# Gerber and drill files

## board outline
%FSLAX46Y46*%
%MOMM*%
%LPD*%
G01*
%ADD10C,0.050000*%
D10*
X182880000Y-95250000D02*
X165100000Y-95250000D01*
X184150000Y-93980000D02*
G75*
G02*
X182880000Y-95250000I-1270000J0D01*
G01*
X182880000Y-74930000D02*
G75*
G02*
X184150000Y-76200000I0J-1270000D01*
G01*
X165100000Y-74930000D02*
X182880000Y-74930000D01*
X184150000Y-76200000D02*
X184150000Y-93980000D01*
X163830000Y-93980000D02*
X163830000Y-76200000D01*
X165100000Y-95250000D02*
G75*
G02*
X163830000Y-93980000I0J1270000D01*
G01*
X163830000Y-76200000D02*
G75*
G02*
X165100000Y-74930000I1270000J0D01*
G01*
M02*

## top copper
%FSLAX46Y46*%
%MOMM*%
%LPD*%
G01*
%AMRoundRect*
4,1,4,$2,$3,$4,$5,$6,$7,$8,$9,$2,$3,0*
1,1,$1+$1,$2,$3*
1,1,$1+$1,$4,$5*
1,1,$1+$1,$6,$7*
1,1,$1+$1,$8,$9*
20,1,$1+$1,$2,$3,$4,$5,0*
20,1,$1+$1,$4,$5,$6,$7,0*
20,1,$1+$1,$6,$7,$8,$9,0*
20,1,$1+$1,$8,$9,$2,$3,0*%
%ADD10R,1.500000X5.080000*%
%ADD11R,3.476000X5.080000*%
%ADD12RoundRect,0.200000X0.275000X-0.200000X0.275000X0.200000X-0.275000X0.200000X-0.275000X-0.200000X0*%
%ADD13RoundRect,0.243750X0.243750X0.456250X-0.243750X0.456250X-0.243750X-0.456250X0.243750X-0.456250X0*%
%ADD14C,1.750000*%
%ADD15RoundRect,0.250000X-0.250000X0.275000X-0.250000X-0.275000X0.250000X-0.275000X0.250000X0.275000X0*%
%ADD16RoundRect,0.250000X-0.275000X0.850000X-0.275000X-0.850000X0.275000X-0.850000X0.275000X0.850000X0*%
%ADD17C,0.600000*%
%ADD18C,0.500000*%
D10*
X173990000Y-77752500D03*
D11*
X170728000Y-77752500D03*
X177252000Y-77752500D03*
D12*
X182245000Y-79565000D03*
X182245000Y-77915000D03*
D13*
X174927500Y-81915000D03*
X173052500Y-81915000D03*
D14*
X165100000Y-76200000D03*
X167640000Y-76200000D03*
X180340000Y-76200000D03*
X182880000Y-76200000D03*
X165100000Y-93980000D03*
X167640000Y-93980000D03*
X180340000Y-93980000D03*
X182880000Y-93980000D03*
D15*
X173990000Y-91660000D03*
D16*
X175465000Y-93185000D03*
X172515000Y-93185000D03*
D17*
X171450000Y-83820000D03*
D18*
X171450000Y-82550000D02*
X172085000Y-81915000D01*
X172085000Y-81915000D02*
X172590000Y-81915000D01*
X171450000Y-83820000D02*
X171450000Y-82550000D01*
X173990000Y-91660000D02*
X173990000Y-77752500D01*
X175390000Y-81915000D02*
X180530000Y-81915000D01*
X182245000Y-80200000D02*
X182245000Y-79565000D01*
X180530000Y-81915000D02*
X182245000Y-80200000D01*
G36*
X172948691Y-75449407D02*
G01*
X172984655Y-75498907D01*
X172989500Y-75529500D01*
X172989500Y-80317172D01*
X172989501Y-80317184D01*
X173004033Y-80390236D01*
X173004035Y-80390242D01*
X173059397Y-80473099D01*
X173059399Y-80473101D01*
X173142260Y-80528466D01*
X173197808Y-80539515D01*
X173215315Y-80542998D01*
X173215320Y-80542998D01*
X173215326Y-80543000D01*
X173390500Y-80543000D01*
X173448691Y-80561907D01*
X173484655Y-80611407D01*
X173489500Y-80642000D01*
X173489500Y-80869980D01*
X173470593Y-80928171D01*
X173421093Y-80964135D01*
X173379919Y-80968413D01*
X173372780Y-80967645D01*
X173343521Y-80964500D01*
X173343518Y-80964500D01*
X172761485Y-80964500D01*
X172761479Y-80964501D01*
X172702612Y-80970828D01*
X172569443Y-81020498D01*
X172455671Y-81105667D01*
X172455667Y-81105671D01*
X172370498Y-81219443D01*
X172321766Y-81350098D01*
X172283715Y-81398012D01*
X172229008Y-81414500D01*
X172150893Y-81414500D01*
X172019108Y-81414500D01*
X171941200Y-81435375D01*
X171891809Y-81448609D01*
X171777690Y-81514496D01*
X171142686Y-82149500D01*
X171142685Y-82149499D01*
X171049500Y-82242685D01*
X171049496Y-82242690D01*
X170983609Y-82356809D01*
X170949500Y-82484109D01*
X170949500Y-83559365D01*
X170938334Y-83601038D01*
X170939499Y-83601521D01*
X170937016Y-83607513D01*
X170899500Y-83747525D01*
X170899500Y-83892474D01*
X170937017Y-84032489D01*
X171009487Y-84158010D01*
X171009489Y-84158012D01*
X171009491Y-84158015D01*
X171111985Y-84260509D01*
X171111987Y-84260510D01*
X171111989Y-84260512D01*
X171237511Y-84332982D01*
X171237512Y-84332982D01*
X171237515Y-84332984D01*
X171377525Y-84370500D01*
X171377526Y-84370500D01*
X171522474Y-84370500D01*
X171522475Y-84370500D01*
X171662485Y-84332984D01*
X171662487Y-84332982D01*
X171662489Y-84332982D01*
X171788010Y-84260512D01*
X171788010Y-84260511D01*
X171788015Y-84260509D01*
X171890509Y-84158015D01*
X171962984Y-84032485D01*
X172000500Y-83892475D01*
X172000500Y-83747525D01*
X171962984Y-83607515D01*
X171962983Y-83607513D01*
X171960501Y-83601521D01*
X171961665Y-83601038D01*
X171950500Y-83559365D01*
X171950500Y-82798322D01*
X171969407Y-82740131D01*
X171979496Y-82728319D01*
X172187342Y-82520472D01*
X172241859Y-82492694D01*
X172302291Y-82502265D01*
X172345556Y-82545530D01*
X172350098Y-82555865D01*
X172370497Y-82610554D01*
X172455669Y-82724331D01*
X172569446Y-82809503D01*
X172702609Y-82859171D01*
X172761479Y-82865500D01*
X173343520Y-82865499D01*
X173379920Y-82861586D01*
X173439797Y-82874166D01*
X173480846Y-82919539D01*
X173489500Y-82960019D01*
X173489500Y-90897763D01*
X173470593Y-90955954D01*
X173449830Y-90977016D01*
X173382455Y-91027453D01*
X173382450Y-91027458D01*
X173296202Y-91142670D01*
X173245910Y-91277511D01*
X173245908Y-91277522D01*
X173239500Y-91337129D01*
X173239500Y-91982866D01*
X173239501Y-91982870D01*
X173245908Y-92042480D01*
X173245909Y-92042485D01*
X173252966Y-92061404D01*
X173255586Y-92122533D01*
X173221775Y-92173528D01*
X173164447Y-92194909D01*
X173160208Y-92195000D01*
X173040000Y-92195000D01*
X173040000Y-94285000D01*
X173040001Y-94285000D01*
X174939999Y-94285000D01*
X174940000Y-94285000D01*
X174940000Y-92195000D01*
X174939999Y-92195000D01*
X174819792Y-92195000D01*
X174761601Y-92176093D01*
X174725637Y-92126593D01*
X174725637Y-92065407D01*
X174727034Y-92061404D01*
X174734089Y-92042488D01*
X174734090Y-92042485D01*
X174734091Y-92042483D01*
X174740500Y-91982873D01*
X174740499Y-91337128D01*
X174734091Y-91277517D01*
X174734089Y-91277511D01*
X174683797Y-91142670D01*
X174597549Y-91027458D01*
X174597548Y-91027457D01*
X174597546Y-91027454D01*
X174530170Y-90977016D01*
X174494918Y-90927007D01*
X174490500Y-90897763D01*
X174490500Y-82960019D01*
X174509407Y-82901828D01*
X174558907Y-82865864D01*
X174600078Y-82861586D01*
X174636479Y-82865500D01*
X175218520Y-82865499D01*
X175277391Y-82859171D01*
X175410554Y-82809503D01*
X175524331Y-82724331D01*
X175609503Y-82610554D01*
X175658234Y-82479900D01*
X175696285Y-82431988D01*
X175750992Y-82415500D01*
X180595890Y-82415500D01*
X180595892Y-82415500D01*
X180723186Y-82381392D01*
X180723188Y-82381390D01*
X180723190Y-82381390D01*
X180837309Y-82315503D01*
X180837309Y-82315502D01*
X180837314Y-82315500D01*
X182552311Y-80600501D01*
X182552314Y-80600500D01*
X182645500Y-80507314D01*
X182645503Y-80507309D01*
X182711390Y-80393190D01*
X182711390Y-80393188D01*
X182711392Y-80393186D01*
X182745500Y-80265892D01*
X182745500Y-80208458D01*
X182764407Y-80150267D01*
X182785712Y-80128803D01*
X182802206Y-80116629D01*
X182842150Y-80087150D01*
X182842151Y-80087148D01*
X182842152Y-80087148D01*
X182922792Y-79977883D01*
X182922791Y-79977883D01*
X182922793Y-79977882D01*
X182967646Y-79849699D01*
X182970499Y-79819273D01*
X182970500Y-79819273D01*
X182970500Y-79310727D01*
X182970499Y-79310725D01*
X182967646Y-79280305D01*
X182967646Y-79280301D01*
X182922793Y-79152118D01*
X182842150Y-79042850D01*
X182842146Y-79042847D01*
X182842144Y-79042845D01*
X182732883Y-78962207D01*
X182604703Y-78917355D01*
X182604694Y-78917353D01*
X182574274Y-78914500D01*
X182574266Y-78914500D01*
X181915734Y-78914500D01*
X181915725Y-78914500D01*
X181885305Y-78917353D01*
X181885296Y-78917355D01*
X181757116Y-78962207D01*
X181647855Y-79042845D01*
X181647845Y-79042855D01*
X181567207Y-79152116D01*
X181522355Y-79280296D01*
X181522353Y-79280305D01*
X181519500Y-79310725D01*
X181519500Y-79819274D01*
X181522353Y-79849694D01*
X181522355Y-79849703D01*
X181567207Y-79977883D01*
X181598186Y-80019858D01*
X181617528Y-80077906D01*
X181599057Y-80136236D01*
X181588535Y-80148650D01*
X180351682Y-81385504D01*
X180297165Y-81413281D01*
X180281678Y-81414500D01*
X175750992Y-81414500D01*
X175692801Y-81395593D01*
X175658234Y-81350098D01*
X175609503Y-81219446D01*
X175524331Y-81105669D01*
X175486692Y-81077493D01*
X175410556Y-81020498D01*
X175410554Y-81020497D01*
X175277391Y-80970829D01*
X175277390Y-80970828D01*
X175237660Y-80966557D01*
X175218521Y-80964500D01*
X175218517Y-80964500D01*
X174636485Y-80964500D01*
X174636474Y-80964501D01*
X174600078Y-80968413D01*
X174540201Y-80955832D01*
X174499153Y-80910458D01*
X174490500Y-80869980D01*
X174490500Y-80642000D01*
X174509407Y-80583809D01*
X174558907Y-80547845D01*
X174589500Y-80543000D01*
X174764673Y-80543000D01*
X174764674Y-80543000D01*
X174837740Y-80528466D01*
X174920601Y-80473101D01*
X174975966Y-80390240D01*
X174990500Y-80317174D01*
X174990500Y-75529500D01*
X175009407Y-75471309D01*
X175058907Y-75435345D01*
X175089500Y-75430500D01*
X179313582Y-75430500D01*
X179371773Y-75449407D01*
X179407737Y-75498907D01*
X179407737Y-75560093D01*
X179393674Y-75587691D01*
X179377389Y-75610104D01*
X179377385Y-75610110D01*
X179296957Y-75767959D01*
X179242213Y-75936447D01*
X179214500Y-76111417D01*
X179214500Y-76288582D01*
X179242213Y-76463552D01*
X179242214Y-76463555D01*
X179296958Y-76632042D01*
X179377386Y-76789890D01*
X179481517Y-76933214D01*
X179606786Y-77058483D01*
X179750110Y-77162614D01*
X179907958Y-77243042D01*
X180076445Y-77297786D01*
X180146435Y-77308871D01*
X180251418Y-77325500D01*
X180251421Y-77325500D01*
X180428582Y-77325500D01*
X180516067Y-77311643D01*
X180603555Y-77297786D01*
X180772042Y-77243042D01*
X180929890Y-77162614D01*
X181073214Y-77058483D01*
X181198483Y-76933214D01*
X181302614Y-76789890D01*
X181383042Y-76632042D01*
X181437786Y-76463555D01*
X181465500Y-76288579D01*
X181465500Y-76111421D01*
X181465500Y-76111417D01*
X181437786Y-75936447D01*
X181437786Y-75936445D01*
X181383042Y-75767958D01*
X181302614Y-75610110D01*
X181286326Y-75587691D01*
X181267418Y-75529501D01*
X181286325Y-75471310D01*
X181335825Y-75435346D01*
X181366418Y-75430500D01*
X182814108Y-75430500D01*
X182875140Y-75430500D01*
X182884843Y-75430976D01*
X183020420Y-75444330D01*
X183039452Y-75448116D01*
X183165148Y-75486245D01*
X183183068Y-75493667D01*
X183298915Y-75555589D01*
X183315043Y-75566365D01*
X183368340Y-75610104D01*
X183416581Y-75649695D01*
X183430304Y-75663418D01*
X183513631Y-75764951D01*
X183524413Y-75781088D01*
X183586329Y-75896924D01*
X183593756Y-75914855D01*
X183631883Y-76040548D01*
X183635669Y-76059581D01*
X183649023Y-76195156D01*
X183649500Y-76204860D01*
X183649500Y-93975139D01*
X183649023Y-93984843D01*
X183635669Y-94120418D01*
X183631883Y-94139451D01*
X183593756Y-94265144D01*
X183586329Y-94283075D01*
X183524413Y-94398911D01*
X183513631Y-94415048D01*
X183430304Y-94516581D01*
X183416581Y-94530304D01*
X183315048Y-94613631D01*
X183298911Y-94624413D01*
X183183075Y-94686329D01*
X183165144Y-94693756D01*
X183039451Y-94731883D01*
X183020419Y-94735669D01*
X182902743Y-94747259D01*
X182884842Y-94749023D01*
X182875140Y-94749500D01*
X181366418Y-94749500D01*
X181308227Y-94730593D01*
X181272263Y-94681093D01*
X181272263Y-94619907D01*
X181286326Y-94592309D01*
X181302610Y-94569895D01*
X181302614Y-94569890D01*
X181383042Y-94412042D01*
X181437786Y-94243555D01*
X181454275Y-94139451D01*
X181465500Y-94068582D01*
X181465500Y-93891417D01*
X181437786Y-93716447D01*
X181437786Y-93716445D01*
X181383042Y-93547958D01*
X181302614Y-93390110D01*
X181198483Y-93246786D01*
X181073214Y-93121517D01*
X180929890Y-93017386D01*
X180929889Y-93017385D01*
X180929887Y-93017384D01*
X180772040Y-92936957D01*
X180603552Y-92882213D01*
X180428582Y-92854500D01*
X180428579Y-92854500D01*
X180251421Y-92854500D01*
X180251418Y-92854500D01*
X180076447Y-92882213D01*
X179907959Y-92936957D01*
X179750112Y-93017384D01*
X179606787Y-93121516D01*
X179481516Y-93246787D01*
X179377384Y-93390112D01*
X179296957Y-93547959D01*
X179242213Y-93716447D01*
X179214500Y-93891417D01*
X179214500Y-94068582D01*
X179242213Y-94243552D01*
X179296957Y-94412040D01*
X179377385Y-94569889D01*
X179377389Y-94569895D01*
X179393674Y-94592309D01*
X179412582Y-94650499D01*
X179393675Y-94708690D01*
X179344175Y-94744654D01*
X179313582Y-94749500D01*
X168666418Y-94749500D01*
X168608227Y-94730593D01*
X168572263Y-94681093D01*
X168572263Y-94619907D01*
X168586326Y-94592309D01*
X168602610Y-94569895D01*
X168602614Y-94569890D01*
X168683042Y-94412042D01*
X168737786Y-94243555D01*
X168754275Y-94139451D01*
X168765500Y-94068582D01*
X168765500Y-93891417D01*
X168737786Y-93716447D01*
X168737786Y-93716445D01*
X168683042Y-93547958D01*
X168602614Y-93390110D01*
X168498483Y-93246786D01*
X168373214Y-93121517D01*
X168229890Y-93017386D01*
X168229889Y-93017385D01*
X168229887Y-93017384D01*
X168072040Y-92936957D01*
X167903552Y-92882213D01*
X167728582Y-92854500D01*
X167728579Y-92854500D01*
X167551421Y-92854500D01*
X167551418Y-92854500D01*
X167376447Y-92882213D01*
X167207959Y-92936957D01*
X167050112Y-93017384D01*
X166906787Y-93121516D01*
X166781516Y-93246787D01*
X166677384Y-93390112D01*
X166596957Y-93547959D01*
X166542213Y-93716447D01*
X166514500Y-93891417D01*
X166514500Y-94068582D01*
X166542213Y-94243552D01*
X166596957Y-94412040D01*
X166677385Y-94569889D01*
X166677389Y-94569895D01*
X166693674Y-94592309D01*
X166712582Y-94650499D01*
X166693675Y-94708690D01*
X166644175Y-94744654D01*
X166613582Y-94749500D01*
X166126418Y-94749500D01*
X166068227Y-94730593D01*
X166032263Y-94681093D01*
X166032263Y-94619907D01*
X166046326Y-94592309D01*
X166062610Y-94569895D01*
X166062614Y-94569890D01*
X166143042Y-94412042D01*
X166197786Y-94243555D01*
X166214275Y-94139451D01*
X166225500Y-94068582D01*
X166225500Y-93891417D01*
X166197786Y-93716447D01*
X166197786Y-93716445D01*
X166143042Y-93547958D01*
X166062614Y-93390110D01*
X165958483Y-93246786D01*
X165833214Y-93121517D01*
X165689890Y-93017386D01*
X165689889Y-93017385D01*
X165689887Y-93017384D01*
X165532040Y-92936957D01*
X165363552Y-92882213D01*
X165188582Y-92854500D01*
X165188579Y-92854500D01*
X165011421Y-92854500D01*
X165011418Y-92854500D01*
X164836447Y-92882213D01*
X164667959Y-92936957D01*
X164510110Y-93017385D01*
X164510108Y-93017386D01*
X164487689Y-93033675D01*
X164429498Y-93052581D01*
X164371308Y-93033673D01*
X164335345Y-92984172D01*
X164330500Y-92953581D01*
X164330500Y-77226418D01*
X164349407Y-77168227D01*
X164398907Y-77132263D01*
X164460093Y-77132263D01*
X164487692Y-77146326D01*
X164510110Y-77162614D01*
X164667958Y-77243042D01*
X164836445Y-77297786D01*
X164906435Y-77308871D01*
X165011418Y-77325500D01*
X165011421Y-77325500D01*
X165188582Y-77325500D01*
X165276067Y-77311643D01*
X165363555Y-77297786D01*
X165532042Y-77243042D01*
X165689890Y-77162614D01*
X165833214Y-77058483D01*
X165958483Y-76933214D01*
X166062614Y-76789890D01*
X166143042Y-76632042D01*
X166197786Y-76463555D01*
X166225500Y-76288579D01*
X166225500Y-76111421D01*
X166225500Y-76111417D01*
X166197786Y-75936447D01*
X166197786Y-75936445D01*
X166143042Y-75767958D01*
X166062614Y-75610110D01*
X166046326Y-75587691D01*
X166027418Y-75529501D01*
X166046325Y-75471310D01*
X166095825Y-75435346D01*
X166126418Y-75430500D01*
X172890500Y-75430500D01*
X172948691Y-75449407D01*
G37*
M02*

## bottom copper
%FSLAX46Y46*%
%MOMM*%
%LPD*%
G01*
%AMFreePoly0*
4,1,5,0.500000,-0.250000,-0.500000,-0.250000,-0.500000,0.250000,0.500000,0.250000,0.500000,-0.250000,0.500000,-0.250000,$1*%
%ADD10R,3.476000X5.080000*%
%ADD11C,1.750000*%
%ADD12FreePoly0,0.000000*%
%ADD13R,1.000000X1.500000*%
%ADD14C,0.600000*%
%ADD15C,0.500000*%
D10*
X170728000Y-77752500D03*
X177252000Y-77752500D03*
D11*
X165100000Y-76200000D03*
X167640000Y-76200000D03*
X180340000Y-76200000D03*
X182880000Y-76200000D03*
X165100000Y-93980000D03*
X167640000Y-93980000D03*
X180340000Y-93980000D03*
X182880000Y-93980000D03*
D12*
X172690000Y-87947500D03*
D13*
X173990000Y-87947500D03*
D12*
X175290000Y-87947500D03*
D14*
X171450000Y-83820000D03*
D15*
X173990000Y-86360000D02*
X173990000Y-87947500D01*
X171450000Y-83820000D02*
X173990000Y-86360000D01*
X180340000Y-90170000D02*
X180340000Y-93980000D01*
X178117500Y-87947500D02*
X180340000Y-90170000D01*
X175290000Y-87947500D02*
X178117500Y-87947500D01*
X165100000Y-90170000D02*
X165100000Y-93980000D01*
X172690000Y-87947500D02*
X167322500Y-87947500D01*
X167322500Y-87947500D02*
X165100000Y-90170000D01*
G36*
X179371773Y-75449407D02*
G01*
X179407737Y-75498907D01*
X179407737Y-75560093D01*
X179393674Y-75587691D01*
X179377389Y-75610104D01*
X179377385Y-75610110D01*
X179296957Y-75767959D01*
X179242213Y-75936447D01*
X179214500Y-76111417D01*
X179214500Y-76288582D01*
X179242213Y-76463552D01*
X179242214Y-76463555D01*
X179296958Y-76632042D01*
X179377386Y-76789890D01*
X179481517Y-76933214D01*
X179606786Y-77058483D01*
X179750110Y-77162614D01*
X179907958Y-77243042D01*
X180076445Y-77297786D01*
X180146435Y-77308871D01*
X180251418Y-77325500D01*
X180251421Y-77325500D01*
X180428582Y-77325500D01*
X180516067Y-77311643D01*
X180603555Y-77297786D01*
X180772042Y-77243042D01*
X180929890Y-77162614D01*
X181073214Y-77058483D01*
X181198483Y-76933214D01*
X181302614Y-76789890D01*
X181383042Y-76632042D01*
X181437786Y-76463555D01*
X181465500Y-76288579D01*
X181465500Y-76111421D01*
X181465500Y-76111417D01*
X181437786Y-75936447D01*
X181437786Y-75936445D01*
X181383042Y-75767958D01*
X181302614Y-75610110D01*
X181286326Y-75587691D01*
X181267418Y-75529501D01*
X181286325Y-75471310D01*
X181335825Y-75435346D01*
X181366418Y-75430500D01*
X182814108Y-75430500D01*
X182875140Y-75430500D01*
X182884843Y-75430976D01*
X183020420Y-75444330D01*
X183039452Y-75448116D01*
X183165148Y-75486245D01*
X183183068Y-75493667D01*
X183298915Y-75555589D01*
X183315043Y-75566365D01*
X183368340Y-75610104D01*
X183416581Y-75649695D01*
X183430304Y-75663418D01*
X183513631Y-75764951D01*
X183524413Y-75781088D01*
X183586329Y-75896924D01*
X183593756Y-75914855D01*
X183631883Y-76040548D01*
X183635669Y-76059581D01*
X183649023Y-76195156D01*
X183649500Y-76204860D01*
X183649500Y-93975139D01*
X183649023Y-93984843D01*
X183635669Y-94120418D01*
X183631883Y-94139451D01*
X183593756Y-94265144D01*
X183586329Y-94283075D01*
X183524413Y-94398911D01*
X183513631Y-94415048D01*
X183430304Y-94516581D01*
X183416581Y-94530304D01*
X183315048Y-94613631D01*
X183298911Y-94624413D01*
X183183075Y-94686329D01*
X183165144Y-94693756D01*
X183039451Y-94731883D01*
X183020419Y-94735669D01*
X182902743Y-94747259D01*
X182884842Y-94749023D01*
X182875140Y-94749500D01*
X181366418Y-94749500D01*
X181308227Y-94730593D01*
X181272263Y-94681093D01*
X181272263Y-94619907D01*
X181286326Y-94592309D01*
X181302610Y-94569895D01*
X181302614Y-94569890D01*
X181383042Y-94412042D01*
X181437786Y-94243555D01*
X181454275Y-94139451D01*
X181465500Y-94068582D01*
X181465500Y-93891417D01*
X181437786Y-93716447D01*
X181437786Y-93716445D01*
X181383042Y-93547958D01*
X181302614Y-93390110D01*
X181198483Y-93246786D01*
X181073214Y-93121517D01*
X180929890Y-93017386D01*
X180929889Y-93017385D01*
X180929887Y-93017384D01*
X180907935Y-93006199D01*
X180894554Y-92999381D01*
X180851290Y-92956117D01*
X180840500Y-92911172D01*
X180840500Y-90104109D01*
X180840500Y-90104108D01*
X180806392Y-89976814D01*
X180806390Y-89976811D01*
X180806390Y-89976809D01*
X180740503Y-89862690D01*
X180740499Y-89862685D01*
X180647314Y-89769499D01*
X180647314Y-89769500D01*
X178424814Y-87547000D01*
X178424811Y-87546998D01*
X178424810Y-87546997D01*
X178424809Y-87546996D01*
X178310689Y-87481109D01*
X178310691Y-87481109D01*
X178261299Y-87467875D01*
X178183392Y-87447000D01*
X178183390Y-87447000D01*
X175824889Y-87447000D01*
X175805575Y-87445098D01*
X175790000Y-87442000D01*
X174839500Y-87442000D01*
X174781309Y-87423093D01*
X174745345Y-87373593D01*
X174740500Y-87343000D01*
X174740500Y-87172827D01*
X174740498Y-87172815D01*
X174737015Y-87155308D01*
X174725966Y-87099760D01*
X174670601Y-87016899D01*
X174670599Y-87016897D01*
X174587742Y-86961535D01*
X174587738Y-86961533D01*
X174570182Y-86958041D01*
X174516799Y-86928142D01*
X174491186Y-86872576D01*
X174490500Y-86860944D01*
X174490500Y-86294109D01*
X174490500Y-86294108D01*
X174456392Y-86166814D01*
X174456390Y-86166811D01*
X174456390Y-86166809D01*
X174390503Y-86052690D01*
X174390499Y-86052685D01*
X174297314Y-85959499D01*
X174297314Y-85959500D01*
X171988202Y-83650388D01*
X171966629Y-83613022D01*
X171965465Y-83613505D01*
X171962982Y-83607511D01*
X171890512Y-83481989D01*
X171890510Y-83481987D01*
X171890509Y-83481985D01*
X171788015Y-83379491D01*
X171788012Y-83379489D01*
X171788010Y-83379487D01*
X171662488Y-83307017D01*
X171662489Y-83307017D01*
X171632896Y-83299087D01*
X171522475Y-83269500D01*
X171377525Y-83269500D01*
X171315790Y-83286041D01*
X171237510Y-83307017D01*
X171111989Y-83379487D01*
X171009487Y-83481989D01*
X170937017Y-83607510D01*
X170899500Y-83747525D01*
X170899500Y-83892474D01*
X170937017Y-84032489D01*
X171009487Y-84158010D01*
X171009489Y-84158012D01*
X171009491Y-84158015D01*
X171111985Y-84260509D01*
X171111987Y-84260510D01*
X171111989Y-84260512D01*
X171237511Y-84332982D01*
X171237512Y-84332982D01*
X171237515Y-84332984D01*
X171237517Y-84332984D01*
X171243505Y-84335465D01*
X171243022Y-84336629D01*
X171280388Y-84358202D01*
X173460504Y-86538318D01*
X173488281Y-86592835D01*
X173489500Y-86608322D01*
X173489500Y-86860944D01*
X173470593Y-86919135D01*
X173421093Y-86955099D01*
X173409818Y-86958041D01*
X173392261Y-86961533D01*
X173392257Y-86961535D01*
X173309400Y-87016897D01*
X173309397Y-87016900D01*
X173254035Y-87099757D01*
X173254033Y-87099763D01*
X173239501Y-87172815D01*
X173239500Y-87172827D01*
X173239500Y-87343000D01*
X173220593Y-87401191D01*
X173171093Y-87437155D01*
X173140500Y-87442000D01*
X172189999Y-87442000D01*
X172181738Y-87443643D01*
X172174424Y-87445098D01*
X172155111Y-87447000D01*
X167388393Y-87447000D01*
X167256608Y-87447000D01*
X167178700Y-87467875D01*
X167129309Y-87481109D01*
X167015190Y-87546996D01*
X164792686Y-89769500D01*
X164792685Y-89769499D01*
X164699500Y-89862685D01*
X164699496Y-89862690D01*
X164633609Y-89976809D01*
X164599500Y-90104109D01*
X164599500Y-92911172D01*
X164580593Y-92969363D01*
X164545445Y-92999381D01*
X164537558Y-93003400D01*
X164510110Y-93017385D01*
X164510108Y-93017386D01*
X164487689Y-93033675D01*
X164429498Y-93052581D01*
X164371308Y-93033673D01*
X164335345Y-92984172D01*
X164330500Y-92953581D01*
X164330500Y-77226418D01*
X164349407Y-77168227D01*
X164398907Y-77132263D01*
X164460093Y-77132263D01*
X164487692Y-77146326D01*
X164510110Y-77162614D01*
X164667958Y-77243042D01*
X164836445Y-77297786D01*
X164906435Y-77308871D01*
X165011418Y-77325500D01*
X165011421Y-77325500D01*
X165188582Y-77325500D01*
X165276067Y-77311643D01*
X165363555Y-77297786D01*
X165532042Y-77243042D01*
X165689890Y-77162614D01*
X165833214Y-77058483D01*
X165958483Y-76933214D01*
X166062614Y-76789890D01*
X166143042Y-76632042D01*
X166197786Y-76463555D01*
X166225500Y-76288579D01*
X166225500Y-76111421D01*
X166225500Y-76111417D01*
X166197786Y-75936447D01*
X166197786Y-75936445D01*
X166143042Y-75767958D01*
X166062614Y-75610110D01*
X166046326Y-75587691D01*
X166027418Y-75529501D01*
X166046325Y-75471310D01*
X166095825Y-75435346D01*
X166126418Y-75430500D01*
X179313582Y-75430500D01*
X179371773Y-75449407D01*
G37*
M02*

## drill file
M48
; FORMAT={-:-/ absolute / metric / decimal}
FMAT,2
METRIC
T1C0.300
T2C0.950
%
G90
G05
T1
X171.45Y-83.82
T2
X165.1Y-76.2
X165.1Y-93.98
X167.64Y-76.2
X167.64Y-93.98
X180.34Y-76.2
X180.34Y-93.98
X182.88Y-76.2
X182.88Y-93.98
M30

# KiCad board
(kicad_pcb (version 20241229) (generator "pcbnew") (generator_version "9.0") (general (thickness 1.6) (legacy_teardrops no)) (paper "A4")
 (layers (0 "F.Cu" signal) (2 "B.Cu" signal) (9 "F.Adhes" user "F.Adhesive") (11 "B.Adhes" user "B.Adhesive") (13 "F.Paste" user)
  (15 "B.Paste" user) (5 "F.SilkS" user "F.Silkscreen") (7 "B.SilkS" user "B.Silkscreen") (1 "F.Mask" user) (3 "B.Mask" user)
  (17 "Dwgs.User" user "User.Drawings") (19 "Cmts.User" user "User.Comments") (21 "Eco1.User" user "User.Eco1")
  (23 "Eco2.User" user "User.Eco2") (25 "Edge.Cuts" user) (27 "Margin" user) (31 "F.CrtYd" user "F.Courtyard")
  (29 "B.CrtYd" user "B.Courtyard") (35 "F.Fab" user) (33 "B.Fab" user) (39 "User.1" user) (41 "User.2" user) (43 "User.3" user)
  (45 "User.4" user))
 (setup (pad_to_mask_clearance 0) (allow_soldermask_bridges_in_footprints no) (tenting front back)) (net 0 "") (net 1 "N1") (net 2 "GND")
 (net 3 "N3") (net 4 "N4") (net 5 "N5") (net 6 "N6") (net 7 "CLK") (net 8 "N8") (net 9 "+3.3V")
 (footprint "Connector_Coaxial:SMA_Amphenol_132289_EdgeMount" (layer "F.Cu") (at 173.99 77.7525 90)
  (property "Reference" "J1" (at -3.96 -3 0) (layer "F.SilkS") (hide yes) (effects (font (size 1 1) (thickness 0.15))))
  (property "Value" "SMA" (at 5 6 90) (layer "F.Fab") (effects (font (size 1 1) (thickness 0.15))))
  (pad "1" smd rect (at 0 0 180) (size 1.5 5.08) (layers "F.Cu" "F.Mask" "F.Paste") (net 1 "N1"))
  (pad "2" smd rect (at 0 -3.262 180) (size 3.476 5.08) (layers "F.Cu" "F.Mask" "F.Paste") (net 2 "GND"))
  (pad "2" smd rect (at 0 -3.262 180) (size 3.476 5.08) (layers "B.Cu" "B.Mask" "B.Paste") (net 2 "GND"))
  (pad "2" smd rect (at 0 3.262 180) (size 3.476 5.08) (layers "F.Cu" "F.Mask" "F.Paste") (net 2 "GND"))
  (pad "2" smd rect (at 0 3.262 180) (size 3.476 5.08) (layers "B.Cu" "B.Mask" "B.Paste") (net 2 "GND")))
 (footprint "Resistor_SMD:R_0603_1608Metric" (layer "F.Cu") (at 182.245 78.74 90)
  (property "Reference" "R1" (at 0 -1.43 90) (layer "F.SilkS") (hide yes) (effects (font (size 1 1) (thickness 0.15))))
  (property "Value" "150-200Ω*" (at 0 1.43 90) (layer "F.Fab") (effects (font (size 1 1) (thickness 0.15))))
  (pad "1" smd roundrect (at -0.825 0 90) (size 0.8 0.95) (layers "F.Cu" "F.Mask" "F.Paste") (roundrect_rratio 0.25) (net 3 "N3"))
  (pad "2" smd roundrect (at 0.825 0 90) (size 0.8 0.95) (layers "F.Cu" "F.Mask" "F.Paste") (roundrect_rratio 0.25) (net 2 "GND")))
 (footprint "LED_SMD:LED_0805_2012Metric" (layer "F.Cu") (at 173.99 81.915 180)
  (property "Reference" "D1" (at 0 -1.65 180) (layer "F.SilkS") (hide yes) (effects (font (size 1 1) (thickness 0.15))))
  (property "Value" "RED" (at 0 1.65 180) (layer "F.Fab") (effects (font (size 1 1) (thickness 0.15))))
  (pad "1" smd roundrect (at -0.9375 0 180) (size 0.975 1.4) (layers "F.Cu" "F.Mask" "F.Paste") (roundrect_rratio 0.25) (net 3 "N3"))
  (pad "2" smd roundrect (at 0.9375 0 180) (size 0.975 1.4) (layers "F.Cu" "F.Mask" "F.Paste") (roundrect_rratio 0.25) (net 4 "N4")))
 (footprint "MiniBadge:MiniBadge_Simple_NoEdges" (layer "F.Cu") (at 163.83 74.93)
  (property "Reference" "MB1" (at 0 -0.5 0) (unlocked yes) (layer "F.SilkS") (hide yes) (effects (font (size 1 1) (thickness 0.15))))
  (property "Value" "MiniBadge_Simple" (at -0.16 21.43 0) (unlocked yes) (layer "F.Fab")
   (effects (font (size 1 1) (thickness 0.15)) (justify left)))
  (pad "1" thru_hole circle (at 1.27 1.27) (size 1.75 1.75) (drill 0.95) (layers "*.Cu" "*.Mask") (remove_unused_layers no) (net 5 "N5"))
  (pad "2" thru_hole circle (at 3.81 1.27) (size 1.75 1.75) (drill 0.95) (layers "*.Cu" "*.Mask") (remove_unused_layers no) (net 2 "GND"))
  (pad "7" thru_hole circle (at 16.51 1.27) (size 1.75 1.75) (drill 0.95) (layers "*.Cu" "*.Mask") (remove_unused_layers no) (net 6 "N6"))
  (pad "8" thru_hole circle (at 19.05 1.27) (size 1.75 1.75) (drill 0.95) (layers "*.Cu" "*.Mask") (remove_unused_layers no) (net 2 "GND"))
  (pad "9" thru_hole circle (at 1.27 19.05) (size 1.75 1.75) (drill 0.95) (layers "*.Cu" "*.Mask") (remove_unused_layers no) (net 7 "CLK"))
  (pad "10" thru_hole circle (at 3.81 19.05) (size 1.75 1.75) (drill 0.95) (layers "*.Cu" "*.Mask") (remove_unused_layers no) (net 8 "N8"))
  (pad "15" thru_hole circle (at 16.51 19.05) (size 1.75 1.75) (drill 0.95) (layers "*.Cu" "*.Mask") (remove_unused_layers no)
   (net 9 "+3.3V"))
  (pad "16" thru_hole circle (at 19.05 19.05) (size 1.75 1.75) (drill 0.95) (layers "*.Cu" "*.Mask") (remove_unused_layers no) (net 2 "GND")))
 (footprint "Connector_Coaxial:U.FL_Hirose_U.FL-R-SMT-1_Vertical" (layer "F.Cu") (at 173.99 92.71 -90)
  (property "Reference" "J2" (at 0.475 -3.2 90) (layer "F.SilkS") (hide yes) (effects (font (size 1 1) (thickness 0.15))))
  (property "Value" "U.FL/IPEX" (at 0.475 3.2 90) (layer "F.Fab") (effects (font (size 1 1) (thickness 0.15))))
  (pad "1" smd roundrect (at -1.05 0 270) (size 1.05 1) (layers "F.Cu" "F.Mask" "F.Paste") (roundrect_rratio 0.25) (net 1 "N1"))
  (pad "2" smd roundrect (at 0.475 -1.475 270) (size 2.2 1.05) (layers "F.Cu" "F.Mask" "F.Paste") (roundrect_rratio 0.2380952381)
   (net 2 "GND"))
  (pad "2" smd roundrect (at 0.475 1.475 270) (size 2.2 1.05) (layers "F.Cu" "F.Mask" "F.Paste") (roundrect_rratio 0.2380952381)
   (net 2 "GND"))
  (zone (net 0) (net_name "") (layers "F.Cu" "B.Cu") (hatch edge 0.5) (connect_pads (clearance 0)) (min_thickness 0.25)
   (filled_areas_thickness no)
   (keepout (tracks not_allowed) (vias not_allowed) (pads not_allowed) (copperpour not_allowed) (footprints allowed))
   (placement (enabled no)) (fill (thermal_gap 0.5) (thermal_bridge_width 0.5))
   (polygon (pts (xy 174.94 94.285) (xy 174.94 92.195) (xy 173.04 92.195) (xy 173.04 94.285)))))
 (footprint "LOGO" (layer "F.Cu") (at 173.99 82.55)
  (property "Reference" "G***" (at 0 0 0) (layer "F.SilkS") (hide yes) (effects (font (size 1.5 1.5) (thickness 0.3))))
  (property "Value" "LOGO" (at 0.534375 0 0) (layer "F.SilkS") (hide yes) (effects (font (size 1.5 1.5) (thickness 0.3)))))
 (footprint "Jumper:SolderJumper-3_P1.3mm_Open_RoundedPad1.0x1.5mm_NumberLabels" (layer "B.Cu") (at 173.99 87.9475)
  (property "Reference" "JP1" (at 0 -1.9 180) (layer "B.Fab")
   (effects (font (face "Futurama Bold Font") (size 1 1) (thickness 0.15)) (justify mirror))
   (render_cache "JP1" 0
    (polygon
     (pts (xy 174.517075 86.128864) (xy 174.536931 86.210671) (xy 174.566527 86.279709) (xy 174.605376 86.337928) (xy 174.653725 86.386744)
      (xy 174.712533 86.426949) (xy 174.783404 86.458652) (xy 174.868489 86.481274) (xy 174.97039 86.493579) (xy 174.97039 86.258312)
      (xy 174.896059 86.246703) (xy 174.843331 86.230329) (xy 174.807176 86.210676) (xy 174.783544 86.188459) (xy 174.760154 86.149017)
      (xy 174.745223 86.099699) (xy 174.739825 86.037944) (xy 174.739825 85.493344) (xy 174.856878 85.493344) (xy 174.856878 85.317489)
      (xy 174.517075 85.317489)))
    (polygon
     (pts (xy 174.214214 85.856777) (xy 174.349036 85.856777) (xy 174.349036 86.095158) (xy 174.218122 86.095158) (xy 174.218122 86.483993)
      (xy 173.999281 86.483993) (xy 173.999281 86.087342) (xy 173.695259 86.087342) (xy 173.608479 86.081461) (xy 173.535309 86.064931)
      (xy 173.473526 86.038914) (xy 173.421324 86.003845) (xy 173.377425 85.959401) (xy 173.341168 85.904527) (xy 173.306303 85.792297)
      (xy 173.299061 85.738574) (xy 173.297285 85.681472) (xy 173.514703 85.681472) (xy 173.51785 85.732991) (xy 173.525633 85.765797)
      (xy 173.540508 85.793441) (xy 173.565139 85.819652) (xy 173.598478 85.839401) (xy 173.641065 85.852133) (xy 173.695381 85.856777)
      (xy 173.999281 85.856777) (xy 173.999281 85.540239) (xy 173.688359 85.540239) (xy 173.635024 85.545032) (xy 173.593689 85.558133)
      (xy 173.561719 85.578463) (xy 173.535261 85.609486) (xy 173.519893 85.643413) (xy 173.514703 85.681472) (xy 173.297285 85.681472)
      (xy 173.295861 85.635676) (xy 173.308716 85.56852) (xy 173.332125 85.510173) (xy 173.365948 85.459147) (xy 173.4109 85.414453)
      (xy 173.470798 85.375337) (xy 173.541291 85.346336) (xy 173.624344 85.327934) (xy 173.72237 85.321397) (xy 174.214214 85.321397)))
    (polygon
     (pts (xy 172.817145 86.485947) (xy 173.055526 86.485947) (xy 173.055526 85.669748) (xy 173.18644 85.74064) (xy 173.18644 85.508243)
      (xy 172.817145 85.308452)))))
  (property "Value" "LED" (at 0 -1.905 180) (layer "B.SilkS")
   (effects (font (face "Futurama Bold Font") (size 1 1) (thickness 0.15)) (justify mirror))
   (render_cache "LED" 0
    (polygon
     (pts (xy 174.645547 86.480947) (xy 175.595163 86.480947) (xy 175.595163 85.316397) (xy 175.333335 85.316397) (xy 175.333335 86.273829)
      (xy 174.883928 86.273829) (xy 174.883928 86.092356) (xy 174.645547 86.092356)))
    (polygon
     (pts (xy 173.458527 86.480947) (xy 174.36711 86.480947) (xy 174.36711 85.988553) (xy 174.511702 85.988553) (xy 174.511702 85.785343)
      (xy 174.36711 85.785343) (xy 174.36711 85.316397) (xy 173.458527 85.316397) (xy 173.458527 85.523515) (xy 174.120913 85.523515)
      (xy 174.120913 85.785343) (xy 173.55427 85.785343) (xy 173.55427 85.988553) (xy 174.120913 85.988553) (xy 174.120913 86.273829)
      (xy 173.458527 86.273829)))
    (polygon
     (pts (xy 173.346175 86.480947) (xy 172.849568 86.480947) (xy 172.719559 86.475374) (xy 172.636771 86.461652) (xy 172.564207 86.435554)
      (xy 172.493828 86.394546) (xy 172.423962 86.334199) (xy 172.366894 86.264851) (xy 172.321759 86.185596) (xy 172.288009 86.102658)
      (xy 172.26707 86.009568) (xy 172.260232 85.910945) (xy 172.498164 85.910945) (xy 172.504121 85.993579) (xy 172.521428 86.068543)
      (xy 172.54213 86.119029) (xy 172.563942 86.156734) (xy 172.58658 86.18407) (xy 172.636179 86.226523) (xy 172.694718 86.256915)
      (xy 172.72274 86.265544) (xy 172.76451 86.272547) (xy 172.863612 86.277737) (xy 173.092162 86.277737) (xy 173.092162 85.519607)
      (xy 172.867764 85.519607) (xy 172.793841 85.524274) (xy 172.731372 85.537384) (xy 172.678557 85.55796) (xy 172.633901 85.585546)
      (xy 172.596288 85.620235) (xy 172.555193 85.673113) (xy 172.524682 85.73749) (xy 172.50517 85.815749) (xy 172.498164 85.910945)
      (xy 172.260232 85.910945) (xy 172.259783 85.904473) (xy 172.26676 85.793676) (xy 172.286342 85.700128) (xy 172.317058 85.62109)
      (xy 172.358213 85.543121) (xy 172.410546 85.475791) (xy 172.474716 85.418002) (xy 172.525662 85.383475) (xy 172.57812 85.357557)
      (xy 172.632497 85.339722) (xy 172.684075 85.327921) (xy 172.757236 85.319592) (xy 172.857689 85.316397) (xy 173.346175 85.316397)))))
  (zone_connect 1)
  (pad "1" smd custom (at -1.3 0) (size 1 0.5) (layers "B.Cu" "B.Mask") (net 7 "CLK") (zone_connect 2) (thermal_bridge_angle 45)
   (options (clearance outline) (anchor rect)) (primitives))
  (pad "2" smd rect (at 0 0) (size 1 1.5) (layers "B.Cu" "B.Mask") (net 4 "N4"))
  (pad "3" smd custom (at 1.3 0) (size 1 0.5) (layers "B.Cu" "B.Mask") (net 9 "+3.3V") (zone_connect 2) (thermal_bridge_angle 45)
   (options (clearance outline) (anchor rect)) (primitives)))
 (gr_line (start 182.88 95.25) (end 165.1 95.25) (stroke (width 0.05) (type default)) (layer "Edge.Cuts"))
 (gr_arc (start 184.15 93.98) (mid 183.778026 94.878026) (end 182.88 95.25) (stroke (width 0.05) (type default)) (layer "Edge.Cuts"))
 (gr_arc (start 182.88 74.93) (mid 183.778026 75.301974) (end 184.15 76.2) (stroke (width 0.05) (type default)) (layer "Edge.Cuts"))
 (gr_line (start 165.1 74.93) (end 182.88 74.93) (stroke (width 0.05) (type default)) (layer "Edge.Cuts"))
 (gr_line (start 184.15 76.2) (end 184.15 93.98) (stroke (width 0.05) (type default)) (layer "Edge.Cuts"))
 (gr_line (start 163.83 93.98) (end 163.83 76.2) (stroke (width 0.05) (type default)) (layer "Edge.Cuts"))
 (gr_arc (start 165.1 95.25) (mid 164.201974 94.878026) (end 163.83 93.98) (stroke (width 0.05) (type default)) (layer "Edge.Cuts"))
 (gr_arc (start 163.83 76.2) (mid 164.201974 75.301974) (end 165.1 74.93) (stroke (width 0.05) (type default)) (layer "Edge.Cuts"))
 (segment (start 171.45 82.55) (end 172.085 81.915) (width 0.5) (layer "F.Cu") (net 4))
 (segment (start 172.085 81.915) (end 172.59 81.915) (width 0.5) (layer "F.Cu") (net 4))
 (segment (start 171.45 83.82) (end 171.45 82.55) (width 0.5) (layer "F.Cu") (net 4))
 (via (at 171.45 83.82) (size 0.6) (drill 0.3) (layers "F.Cu" "B.Cu") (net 4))
 (segment (start 173.99 86.36) (end 173.99 87.9475) (width 0.5) (layer "B.Cu") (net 4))
 (segment (start 171.45 83.82) (end 173.99 86.36) (width 0.5) (layer "B.Cu") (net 4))
 (segment (start 173.99 91.66) (end 173.99 77.7525) (width 0.5) (layer "F.Cu") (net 1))
 (segment (start 180.34 90.17) (end 180.34 93.98) (width 0.5) (layer "B.Cu") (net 9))
 (segment (start 178.1175 87.9475) (end 180.34 90.17) (width 0.5) (layer "B.Cu") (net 9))
 (segment (start 175.29 87.9475) (end 178.1175 87.9475) (width 0.5) (layer "B.Cu") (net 9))
 (segment (start 165.1 90.17) (end 165.1 93.98) (width 0.5) (layer "B.Cu") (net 7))
 (segment (start 172.69 87.9475) (end 167.3225 87.9475) (width 0.5) (layer "B.Cu") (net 7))
 (segment (start 167.3225 87.9475) (end 165.1 90.17) (width 0.5) (layer "B.Cu") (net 7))
 (segment (start 175.39 81.915) (end 180.53 81.915) (width 0.5) (layer "F.Cu") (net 3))
 (segment (start 182.245 80.2) (end 182.245 79.565) (width 0.5) (layer "F.Cu") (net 3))
 (segment (start 180.53 81.915) (end 182.245 80.2) (width 0.5) (layer "F.Cu") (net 3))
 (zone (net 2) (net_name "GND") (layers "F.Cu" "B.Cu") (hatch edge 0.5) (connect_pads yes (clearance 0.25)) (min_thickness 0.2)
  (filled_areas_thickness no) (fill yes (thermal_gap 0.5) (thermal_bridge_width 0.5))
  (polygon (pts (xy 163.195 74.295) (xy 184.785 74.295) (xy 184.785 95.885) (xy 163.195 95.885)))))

